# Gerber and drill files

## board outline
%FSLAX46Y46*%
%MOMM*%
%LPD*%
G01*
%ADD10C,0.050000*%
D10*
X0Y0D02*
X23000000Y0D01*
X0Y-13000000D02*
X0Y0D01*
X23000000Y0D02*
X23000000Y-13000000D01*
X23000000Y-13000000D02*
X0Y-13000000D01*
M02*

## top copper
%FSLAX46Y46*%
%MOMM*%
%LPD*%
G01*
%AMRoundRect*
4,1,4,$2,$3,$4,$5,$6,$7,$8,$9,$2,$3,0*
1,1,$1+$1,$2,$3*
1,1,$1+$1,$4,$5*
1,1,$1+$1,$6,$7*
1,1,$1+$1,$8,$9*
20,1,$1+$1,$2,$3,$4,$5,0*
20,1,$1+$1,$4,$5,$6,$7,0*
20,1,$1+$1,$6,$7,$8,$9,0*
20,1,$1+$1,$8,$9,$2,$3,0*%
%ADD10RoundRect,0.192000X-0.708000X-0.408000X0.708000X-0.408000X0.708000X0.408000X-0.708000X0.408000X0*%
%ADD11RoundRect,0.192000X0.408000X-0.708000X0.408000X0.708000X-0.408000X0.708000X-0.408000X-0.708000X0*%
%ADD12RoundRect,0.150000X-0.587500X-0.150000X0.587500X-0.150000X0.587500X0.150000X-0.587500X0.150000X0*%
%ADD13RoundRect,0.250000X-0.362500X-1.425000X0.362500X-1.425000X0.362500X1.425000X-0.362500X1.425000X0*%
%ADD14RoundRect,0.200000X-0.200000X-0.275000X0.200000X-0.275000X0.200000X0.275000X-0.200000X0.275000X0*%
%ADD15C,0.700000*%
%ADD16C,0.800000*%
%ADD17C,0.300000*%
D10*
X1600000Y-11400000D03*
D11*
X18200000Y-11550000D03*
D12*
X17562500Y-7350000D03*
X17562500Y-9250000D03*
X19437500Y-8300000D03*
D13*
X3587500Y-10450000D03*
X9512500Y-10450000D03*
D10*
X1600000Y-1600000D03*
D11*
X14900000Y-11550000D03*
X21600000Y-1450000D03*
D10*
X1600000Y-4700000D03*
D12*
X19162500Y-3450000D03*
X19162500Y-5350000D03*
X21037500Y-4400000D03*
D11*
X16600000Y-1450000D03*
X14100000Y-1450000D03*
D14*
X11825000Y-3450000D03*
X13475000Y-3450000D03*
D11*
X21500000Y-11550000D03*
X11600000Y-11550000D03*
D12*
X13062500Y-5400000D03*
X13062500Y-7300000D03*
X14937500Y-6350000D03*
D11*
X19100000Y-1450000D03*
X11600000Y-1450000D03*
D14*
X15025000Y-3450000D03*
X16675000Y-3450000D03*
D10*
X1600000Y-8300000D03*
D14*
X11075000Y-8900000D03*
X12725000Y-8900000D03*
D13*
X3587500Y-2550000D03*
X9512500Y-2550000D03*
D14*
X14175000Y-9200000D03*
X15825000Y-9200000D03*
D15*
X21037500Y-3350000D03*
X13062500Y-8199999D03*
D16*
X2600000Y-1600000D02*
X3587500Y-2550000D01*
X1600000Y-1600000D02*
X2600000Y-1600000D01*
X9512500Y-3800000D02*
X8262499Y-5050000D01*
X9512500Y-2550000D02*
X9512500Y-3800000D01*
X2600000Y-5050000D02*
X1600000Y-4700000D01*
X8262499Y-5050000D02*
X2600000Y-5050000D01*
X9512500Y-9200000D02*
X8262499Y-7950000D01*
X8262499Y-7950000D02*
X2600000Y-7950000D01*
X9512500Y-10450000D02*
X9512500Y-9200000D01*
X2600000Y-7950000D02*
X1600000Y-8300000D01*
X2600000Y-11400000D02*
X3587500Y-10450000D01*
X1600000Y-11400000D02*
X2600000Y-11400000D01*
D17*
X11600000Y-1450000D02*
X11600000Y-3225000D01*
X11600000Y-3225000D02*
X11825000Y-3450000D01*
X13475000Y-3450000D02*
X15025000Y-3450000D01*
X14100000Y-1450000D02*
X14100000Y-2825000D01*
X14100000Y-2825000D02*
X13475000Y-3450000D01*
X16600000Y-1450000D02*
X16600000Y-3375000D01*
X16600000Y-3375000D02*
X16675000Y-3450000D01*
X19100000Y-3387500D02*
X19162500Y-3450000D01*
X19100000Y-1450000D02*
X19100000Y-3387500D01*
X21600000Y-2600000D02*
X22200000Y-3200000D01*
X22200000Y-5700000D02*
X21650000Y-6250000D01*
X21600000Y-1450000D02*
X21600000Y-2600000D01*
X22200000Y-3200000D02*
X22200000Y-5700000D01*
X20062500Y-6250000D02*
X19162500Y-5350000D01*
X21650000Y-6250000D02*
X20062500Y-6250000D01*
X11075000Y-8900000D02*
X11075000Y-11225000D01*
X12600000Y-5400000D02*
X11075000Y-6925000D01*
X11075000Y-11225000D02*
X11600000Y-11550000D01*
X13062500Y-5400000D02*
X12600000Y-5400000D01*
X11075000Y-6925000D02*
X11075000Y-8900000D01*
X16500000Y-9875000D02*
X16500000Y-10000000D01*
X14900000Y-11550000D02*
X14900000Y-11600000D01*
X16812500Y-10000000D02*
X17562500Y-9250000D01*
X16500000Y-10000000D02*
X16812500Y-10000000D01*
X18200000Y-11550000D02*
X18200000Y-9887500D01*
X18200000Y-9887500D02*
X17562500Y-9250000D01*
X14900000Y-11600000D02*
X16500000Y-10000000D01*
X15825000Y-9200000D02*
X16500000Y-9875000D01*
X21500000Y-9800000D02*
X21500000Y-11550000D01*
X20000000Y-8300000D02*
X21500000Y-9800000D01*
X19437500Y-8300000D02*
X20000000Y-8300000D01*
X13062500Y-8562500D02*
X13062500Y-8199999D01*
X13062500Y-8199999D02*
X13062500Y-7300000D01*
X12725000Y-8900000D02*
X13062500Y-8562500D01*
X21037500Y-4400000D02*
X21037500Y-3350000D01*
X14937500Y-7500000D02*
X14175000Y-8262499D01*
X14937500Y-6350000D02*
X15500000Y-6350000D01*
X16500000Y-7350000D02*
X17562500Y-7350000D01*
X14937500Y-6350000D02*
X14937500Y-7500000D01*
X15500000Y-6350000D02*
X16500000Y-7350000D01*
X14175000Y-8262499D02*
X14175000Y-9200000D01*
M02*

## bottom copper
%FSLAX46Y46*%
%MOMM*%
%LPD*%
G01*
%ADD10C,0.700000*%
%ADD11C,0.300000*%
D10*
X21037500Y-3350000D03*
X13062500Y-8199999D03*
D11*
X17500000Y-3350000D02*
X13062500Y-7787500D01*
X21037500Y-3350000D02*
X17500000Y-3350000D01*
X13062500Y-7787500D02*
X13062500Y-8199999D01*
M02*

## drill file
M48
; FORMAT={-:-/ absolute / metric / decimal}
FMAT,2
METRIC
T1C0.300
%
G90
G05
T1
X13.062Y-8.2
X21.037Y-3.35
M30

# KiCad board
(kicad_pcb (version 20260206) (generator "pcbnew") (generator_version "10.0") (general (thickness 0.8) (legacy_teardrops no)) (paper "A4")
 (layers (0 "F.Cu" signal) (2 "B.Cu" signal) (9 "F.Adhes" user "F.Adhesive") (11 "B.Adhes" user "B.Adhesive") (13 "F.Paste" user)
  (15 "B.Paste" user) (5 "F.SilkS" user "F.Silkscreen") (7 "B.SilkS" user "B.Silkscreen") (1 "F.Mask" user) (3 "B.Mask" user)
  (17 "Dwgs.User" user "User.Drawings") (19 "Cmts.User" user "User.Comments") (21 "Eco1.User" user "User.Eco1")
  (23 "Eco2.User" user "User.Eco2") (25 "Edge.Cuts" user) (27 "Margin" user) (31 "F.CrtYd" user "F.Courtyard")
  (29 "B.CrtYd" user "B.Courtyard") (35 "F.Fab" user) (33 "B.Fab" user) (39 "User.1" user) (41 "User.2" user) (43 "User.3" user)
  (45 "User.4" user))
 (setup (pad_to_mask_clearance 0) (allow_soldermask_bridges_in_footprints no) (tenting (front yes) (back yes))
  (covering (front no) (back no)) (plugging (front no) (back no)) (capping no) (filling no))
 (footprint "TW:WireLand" (layer "F.Cu") (at 1.6 11.4)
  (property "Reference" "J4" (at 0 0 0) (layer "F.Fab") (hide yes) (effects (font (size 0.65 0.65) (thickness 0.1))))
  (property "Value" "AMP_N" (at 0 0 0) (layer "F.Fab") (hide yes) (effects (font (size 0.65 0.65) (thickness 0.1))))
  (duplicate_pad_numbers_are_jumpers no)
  (pad "1" smd roundrect (at 0 0) (size 1.8 1.2) (layers "F.Cu" "F.Mask") (roundrect_rratio 0.16) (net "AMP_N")))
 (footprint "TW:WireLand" (layer "F.Cu") (at 18.2 11.55 90)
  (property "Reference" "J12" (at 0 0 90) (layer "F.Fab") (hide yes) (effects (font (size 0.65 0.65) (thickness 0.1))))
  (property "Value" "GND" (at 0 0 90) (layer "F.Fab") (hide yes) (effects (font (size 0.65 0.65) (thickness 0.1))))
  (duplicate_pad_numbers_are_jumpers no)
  (pad "1" smd roundrect (at 0 0 90) (size 1.8 1.2) (layers "F.Cu" "F.Mask") (roundrect_rratio 0.16) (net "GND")))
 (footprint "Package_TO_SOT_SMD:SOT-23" (layer "F.Cu") (at 18.5 8.3)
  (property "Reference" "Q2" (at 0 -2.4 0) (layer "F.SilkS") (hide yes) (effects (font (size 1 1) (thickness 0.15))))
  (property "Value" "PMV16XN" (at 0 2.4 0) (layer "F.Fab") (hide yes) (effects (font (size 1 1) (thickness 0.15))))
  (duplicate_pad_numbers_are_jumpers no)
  (pad "1" smd roundrect (at -0.9375 -0.95) (size 1.475 0.6) (layers "F.Cu" "F.Mask" "F.Paste") (roundrect_rratio 0.25) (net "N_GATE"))
  (pad "2" smd roundrect (at -0.9375 0.95) (size 1.475 0.6) (layers "F.Cu" "F.Mask" "F.Paste") (roundrect_rratio 0.25) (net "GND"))
  (pad "3" smd roundrect (at 0.9375 0) (size 1.475 0.6) (layers "F.Cu" "F.Mask" "F.Paste") (roundrect_rratio 0.25) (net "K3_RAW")))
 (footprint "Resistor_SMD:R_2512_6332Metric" (layer "F.Cu") (at 6.55 10.45)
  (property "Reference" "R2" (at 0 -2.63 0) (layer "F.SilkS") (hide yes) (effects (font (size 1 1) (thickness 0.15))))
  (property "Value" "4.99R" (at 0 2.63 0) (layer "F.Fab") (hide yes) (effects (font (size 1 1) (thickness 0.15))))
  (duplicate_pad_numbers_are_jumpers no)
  (pad "1" smd roundrect (at -2.9625 0) (size 1.225 3.35) (layers "F.Cu" "F.Mask" "F.Paste") (roundrect_rratio 0.204082) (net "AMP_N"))
  (pad "2" smd roundrect (at 2.9625 0) (size 1.225 3.35) (layers "F.Cu" "F.Mask" "F.Paste") (roundrect_rratio 0.204082) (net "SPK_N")))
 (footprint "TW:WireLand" (layer "F.Cu") (at 1.6 1.6)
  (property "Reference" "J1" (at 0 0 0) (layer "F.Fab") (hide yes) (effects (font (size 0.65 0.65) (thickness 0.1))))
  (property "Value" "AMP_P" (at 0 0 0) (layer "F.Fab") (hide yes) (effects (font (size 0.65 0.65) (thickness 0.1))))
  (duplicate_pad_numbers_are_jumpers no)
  (pad "1" smd roundrect (at 0 0) (size 1.8 1.2) (layers "F.Cu" "F.Mask") (roundrect_rratio 0.16) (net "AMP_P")))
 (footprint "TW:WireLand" (layer "F.Cu") (at 14.9 11.55 90)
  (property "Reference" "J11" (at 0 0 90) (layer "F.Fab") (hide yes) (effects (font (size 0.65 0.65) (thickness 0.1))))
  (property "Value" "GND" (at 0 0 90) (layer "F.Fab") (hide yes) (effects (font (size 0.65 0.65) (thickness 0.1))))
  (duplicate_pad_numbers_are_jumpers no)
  (pad "1" smd roundrect (at 0 0 90) (size 1.8 1.2) (layers "F.Cu" "F.Mask") (roundrect_rratio 0.16) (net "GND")))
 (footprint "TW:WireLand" (layer "F.Cu") (at 21.6 1.45 90)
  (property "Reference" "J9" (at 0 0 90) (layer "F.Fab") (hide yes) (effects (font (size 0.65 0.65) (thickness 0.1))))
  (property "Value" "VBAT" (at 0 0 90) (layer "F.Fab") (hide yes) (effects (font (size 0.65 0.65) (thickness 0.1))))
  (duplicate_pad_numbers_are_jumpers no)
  (pad "1" smd roundrect (at 0 0 90) (size 1.8 1.2) (layers "F.Cu" "F.Mask") (roundrect_rratio 0.16) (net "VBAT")))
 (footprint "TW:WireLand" (layer "F.Cu") (at 1.6 4.7)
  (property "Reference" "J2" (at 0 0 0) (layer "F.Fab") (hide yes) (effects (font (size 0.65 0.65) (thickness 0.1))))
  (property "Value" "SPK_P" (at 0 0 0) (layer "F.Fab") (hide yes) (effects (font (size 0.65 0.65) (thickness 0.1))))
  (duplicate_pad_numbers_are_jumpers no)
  (pad "1" smd roundrect (at 0 0) (size 1.8 1.2) (layers "F.Cu" "F.Mask") (roundrect_rratio 0.16) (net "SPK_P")))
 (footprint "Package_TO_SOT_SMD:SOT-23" (layer "F.Cu") (at 20.1 4.4)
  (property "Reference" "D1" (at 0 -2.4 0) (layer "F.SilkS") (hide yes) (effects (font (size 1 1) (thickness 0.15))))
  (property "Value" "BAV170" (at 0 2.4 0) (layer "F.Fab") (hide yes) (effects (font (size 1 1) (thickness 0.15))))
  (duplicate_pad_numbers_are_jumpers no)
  (pad "1" smd roundrect (at -0.9375 -0.95) (size 1.475 0.6) (layers "F.Cu" "F.Mask" "F.Paste") (roundrect_rratio 0.25) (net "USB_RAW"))
  (pad "2" smd roundrect (at -0.9375 0.95) (size 1.475 0.6) (layers "F.Cu" "F.Mask" "F.Paste") (roundrect_rratio 0.25) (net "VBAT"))
  (pad "3" smd roundrect (at 0.9375 0) (size 1.475 0.6) (layers "F.Cu" "F.Mask" "F.Paste") (roundrect_rratio 0.25) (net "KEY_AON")))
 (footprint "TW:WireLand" (layer "F.Cu") (at 16.6 1.45 90)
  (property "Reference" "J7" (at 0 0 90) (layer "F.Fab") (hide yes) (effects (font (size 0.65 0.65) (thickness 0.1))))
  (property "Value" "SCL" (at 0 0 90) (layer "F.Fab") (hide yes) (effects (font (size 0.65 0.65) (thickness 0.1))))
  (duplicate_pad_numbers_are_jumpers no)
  (pad "1" smd roundrect (at 0 0 90) (size 1.8 1.2) (layers "F.Cu" "F.Mask") (roundrect_rratio 0.16) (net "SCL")))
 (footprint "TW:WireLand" (layer "F.Cu") (at 14.1 1.45 90)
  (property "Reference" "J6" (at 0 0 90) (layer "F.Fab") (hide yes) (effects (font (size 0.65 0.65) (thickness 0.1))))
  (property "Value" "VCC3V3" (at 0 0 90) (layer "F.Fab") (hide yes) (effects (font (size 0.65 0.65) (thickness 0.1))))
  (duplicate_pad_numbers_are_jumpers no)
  (pad "1" smd roundrect (at 0 0 90) (size 1.8 1.2) (layers "F.Cu" "F.Mask") (roundrect_rratio 0.16) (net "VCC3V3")))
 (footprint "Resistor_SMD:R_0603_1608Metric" (layer "F.Cu") (at 12.65 3.45)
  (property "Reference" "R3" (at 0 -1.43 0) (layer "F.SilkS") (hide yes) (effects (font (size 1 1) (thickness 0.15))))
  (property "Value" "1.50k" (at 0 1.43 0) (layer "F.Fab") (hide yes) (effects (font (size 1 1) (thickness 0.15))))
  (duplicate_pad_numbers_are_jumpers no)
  (pad "1" smd roundrect (at -0.825 0) (size 0.8 0.95) (layers "F.Cu" "F.Mask" "F.Paste") (roundrect_rratio 0.25) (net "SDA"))
  (pad "2" smd roundrect (at 0.825 0) (size 0.8 0.95) (layers "F.Cu" "F.Mask" "F.Paste") (roundrect_rratio 0.25) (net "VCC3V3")))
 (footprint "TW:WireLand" (layer "F.Cu") (at 21.5 11.55 90)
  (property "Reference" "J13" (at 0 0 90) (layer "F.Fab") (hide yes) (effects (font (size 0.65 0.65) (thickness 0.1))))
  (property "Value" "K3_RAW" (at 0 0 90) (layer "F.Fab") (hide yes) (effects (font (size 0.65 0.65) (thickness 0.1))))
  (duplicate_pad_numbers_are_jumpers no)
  (pad "1" smd roundrect (at 0 0 90) (size 1.8 1.2) (layers "F.Cu" "F.Mask") (roundrect_rratio 0.16) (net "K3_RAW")))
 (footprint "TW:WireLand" (layer "F.Cu") (at 11.6 11.55 90)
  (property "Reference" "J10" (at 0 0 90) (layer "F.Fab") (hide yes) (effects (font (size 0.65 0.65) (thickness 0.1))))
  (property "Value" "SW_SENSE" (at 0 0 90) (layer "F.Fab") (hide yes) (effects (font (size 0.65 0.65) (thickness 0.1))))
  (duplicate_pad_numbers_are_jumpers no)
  (pad "1" smd roundrect (at 0 0 90) (size 1.8 1.2) (layers "F.Cu" "F.Mask") (roundrect_rratio 0.16) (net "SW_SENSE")))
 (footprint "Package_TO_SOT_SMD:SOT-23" (layer "F.Cu") (at 14 6.35)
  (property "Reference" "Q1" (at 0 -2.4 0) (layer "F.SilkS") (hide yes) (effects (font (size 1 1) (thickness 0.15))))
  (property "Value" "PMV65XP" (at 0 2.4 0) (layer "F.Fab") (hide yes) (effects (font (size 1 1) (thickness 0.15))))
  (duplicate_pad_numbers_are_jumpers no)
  (pad "1" smd roundrect (at -0.9375 -0.95) (size 1.475 0.6) (layers "F.Cu" "F.Mask" "F.Paste") (roundrect_rratio 0.25) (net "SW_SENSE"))
  (pad "2" smd roundrect (at -0.9375 0.95) (size 1.475 0.6) (layers "F.Cu" "F.Mask" "F.Paste") (roundrect_rratio 0.25) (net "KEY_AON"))
  (pad "3" smd roundrect (at 0.9375 0) (size 1.475 0.6) (layers "F.Cu" "F.Mask" "F.Paste") (roundrect_rratio 0.25) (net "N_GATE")))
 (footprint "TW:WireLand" (layer "F.Cu") (at 19.1 1.45 90)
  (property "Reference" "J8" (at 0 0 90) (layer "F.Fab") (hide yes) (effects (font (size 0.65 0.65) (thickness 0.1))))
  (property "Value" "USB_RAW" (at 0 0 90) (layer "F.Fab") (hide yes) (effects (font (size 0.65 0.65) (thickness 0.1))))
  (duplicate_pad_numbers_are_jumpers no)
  (pad "1" smd roundrect (at 0 0 90) (size 1.8 1.2) (layers "F.Cu" "F.Mask") (roundrect_rratio 0.16) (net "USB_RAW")))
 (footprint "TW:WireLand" (layer "F.Cu") (at 11.6 1.45 90)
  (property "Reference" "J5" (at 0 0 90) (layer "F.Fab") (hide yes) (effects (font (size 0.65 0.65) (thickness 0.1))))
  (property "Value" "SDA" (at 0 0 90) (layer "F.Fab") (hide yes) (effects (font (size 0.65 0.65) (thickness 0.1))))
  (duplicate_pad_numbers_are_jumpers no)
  (pad "1" smd roundrect (at 0 0 90) (size 1.8 1.2) (layers "F.Cu" "F.Mask") (roundrect_rratio 0.16) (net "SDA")))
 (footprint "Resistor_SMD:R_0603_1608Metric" (layer "F.Cu") (at 15.85 3.45)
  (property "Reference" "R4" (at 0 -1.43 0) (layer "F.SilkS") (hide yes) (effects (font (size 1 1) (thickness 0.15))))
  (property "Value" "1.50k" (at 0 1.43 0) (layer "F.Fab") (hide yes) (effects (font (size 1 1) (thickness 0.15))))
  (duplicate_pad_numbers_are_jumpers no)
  (pad "1" smd roundrect (at -0.825 0) (size 0.8 0.95) (layers "F.Cu" "F.Mask" "F.Paste") (roundrect_rratio 0.25) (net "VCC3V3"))
  (pad "2" smd roundrect (at 0.825 0) (size 0.8 0.95) (layers "F.Cu" "F.Mask" "F.Paste") (roundrect_rratio 0.25) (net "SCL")))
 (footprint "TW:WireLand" (layer "F.Cu") (at 1.6 8.3)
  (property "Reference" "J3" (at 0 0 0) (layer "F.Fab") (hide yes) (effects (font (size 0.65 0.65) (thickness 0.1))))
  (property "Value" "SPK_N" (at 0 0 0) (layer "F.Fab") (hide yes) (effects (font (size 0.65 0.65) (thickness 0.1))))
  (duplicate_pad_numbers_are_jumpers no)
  (pad "1" smd roundrect (at 0 0) (size 1.8 1.2) (layers "F.Cu" "F.Mask") (roundrect_rratio 0.16) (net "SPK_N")))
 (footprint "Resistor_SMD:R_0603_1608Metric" (layer "F.Cu") (at 11.9 8.9)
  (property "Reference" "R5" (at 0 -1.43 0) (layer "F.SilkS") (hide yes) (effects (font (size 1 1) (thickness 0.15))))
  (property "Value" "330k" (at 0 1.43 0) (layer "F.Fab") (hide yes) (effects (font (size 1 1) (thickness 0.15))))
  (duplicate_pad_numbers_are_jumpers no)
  (pad "1" smd roundrect (at -0.825 0) (size 0.8 0.95) (layers "F.Cu" "F.Mask" "F.Paste") (roundrect_rratio 0.25) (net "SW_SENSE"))
  (pad "2" smd roundrect (at 0.825 0) (size 0.8 0.95) (layers "F.Cu" "F.Mask" "F.Paste") (roundrect_rratio 0.25) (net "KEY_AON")))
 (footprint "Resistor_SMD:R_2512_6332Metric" (layer "F.Cu") (at 6.55 2.55)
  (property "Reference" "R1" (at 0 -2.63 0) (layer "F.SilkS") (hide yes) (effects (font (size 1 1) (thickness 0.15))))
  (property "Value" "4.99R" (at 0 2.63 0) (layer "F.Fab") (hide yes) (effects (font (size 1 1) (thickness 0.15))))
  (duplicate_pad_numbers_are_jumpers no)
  (pad "1" smd roundrect (at -2.9625 0) (size 1.225 3.35) (layers "F.Cu" "F.Mask" "F.Paste") (roundrect_rratio 0.204082) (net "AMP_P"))
  (pad "2" smd roundrect (at 2.9625 0) (size 1.225 3.35) (layers "F.Cu" "F.Mask" "F.Paste") (roundrect_rratio 0.204082) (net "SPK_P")))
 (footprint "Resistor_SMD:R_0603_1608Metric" (layer "F.Cu") (at 15 9.2)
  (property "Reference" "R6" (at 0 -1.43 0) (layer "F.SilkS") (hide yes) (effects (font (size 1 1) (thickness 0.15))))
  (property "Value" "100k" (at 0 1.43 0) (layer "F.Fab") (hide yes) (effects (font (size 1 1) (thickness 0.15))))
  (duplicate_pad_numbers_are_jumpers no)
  (pad "1" smd roundrect (at -0.825 0) (size 0.8 0.95) (layers "F.Cu" "F.Mask" "F.Paste") (roundrect_rratio 0.25) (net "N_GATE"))
  (pad "2" smd roundrect (at 0.825 0) (size 0.8 0.95) (layers "F.Cu" "F.Mask" "F.Paste") (roundrect_rratio 0.25) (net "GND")))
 (gr_line (start 0 0) (end 23 0) (stroke (width 0.05) (type default)) (layer "Edge.Cuts"))
 (gr_line (start 0 13) (end 0 0) (stroke (width 0.05) (type default)) (layer "Edge.Cuts"))
 (gr_line (start 23 0) (end 23 13) (stroke (width 0.05) (type default)) (layer "Edge.Cuts"))
 (gr_line (start 23 13) (end 0 13) (stroke (width 0.05) (type default)) (layer "Edge.Cuts"))
 (segment (start 2.6 1.6) (end 3.5875 2.55) (width 0.8) (layer "F.Cu") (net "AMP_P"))
 (segment (start 1.6 1.6) (end 2.6 1.6) (width 0.8) (layer "F.Cu") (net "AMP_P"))
 (segment (start 9.5125 3.8) (end 8.262499 5.05) (width 0.8) (layer "F.Cu") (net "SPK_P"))
 (segment (start 9.5125 2.55) (end 9.5125 3.8) (width 0.8) (layer "F.Cu") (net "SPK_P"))
 (segment (start 2.6 5.05) (end 1.6 4.7) (width 0.8) (layer "F.Cu") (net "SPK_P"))
 (segment (start 8.262499 5.05) (end 2.6 5.05) (width 0.8) (layer "F.Cu") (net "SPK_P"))
 (segment (start 9.5125 9.2) (end 8.262499 7.95) (width 0.8) (layer "F.Cu") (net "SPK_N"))
 (segment (start 8.262499 7.95) (end 2.6 7.95) (width 0.8) (layer "F.Cu") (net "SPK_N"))
 (segment (start 9.5125 10.45) (end 9.5125 9.2) (width 0.8) (layer "F.Cu") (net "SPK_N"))
 (segment (start 2.6 7.95) (end 1.6 8.3) (width 0.8) (layer "F.Cu") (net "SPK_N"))
 (segment (start 2.6 11.4) (end 3.5875 10.45) (width 0.8) (layer "F.Cu") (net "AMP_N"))
 (segment (start 1.6 11.4) (end 2.6 11.4) (width 0.8) (layer "F.Cu") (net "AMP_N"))
 (segment (start 11.6 1.45) (end 11.6 3.225) (width 0.3) (layer "F.Cu") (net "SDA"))
 (segment (start 11.6 3.225) (end 11.825 3.45) (width 0.3) (layer "F.Cu") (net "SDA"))
 (segment (start 13.475 3.45) (end 15.025 3.45) (width 0.3) (layer "F.Cu") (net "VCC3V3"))
 (segment (start 14.1 1.45) (end 14.1 2.825) (width 0.3) (layer "F.Cu") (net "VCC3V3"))
 (segment (start 14.1 2.825) (end 13.475 3.45) (width 0.3) (layer "F.Cu") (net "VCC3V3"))
 (segment (start 16.6 1.45) (end 16.6 3.375) (width 0.3) (layer "F.Cu") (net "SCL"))
 (segment (start 16.6 3.375) (end 16.675 3.45) (width 0.3) (layer "F.Cu") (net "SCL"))
 (segment (start 19.1 3.3875) (end 19.1625 3.45) (width 0.3) (layer "F.Cu") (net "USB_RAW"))
 (segment (start 19.1 1.45) (end 19.1 3.3875) (width 0.3) (layer "F.Cu") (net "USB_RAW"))
 (segment (start 21.6 2.6) (end 22.2 3.2) (width 0.3) (layer "F.Cu") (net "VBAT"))
 (segment (start 22.2 5.7) (end 21.65 6.25) (width 0.3) (layer "F.Cu") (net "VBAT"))
 (segment (start 21.6 1.45) (end 21.6 2.6) (width 0.3) (layer "F.Cu") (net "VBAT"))
 (segment (start 22.2 3.2) (end 22.2 5.7) (width 0.3) (layer "F.Cu") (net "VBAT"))
 (segment (start 20.0625 6.25) (end 19.1625 5.35) (width 0.3) (layer "F.Cu") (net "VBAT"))
 (segment (start 21.65 6.25) (end 20.0625 6.25) (width 0.3) (layer "F.Cu") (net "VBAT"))
 (segment (start 11.075 8.9) (end 11.075 11.225) (width 0.3) (layer "F.Cu") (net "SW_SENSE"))
 (segment (start 12.6 5.4) (end 11.075 6.925) (width 0.3) (layer "F.Cu") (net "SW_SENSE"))
 (segment (start 11.075 11.225) (end 11.6 11.55) (width 0.3) (layer "F.Cu") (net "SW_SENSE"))
 (segment (start 13.0625 5.4) (end 12.6 5.4) (width 0.3) (layer "F.Cu") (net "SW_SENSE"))
 (segment (start 11.075 6.925) (end 11.075 8.9) (width 0.3) (layer "F.Cu") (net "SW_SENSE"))
 (segment (start 16.5 9.875) (end 16.5 10) (width 0.3) (layer "F.Cu") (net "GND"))
 (segment (start 14.9 11.55) (end 14.9 11.6) (width 0.3) (layer "F.Cu") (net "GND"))
 (segment (start 16.8125 10) (end 17.5625 9.25) (width 0.3) (layer "F.Cu") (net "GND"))
 (segment (start 16.5 10) (end 16.8125 10) (width 0.3) (layer "F.Cu") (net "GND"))
 (segment (start 18.2 11.55) (end 18.2 9.8875) (width 0.3) (layer "F.Cu") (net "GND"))
 (segment (start 18.2 9.8875) (end 17.5625 9.25) (width 0.3) (layer "F.Cu") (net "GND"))
 (segment (start 14.9 11.6) (end 16.5 10) (width 0.3) (layer "F.Cu") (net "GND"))
 (segment (start 15.825 9.2) (end 16.5 9.875) (width 0.3) (layer "F.Cu") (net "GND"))
 (segment (start 21.5 9.8) (end 21.5 11.55) (width 0.3) (layer "F.Cu") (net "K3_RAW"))
 (segment (start 20 8.3) (end 21.5 9.8) (width 0.3) (layer "F.Cu") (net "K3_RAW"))
 (segment (start 19.4375 8.3) (end 20 8.3) (width 0.3) (layer "F.Cu") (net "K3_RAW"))
 (segment (start 13.0625 8.5625) (end 13.0625 8.199999) (width 0.3) (layer "F.Cu") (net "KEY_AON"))
 (segment (start 13.0625 8.199999) (end 13.0625 7.3) (width 0.3) (layer "F.Cu") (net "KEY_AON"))
 (segment (start 12.725 8.9) (end 13.0625 8.5625) (width 0.3) (layer "F.Cu") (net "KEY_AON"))
 (segment (start 21.0375 4.4) (end 21.0375 3.35) (width 0.3) (layer "F.Cu") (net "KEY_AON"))
 (via (at 21.0375 3.35) (size 0.7) (drill 0.3) (layers "F.Cu" "B.Cu") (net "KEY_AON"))
 (via (at 13.0625 8.199999) (size 0.7) (drill 0.3) (layers "F.Cu" "B.Cu") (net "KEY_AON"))
 (segment (start 17.5 3.35) (end 13.0625 7.7875) (width 0.3) (layer "B.Cu") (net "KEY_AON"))
 (segment (start 21.0375 3.35) (end 17.5 3.35) (width 0.3) (layer "B.Cu") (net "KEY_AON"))
 (segment (start 13.0625 7.7875) (end 13.0625 8.199999) (width 0.3) (layer "B.Cu") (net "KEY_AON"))
 (segment (start 14.9375 7.5) (end 14.175 8.262499) (width 0.3) (layer "F.Cu") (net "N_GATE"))
 (segment (start 14.9375 6.35) (end 15.5 6.35) (width 0.3) (layer "F.Cu") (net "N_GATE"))
 (segment (start 16.5 7.35) (end 17.5625 7.35) (width 0.3) (layer "F.Cu") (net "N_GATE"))
 (segment (start 14.9375 6.35) (end 14.9375 7.5) (width 0.3) (layer "F.Cu") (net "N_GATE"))
 (segment (start 15.5 6.35) (end 16.5 7.35) (width 0.3) (layer "F.Cu") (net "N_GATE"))
 (segment (start 14.175 8.262499) (end 14.175 9.2) (width 0.3) (layer "F.Cu") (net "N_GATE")))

